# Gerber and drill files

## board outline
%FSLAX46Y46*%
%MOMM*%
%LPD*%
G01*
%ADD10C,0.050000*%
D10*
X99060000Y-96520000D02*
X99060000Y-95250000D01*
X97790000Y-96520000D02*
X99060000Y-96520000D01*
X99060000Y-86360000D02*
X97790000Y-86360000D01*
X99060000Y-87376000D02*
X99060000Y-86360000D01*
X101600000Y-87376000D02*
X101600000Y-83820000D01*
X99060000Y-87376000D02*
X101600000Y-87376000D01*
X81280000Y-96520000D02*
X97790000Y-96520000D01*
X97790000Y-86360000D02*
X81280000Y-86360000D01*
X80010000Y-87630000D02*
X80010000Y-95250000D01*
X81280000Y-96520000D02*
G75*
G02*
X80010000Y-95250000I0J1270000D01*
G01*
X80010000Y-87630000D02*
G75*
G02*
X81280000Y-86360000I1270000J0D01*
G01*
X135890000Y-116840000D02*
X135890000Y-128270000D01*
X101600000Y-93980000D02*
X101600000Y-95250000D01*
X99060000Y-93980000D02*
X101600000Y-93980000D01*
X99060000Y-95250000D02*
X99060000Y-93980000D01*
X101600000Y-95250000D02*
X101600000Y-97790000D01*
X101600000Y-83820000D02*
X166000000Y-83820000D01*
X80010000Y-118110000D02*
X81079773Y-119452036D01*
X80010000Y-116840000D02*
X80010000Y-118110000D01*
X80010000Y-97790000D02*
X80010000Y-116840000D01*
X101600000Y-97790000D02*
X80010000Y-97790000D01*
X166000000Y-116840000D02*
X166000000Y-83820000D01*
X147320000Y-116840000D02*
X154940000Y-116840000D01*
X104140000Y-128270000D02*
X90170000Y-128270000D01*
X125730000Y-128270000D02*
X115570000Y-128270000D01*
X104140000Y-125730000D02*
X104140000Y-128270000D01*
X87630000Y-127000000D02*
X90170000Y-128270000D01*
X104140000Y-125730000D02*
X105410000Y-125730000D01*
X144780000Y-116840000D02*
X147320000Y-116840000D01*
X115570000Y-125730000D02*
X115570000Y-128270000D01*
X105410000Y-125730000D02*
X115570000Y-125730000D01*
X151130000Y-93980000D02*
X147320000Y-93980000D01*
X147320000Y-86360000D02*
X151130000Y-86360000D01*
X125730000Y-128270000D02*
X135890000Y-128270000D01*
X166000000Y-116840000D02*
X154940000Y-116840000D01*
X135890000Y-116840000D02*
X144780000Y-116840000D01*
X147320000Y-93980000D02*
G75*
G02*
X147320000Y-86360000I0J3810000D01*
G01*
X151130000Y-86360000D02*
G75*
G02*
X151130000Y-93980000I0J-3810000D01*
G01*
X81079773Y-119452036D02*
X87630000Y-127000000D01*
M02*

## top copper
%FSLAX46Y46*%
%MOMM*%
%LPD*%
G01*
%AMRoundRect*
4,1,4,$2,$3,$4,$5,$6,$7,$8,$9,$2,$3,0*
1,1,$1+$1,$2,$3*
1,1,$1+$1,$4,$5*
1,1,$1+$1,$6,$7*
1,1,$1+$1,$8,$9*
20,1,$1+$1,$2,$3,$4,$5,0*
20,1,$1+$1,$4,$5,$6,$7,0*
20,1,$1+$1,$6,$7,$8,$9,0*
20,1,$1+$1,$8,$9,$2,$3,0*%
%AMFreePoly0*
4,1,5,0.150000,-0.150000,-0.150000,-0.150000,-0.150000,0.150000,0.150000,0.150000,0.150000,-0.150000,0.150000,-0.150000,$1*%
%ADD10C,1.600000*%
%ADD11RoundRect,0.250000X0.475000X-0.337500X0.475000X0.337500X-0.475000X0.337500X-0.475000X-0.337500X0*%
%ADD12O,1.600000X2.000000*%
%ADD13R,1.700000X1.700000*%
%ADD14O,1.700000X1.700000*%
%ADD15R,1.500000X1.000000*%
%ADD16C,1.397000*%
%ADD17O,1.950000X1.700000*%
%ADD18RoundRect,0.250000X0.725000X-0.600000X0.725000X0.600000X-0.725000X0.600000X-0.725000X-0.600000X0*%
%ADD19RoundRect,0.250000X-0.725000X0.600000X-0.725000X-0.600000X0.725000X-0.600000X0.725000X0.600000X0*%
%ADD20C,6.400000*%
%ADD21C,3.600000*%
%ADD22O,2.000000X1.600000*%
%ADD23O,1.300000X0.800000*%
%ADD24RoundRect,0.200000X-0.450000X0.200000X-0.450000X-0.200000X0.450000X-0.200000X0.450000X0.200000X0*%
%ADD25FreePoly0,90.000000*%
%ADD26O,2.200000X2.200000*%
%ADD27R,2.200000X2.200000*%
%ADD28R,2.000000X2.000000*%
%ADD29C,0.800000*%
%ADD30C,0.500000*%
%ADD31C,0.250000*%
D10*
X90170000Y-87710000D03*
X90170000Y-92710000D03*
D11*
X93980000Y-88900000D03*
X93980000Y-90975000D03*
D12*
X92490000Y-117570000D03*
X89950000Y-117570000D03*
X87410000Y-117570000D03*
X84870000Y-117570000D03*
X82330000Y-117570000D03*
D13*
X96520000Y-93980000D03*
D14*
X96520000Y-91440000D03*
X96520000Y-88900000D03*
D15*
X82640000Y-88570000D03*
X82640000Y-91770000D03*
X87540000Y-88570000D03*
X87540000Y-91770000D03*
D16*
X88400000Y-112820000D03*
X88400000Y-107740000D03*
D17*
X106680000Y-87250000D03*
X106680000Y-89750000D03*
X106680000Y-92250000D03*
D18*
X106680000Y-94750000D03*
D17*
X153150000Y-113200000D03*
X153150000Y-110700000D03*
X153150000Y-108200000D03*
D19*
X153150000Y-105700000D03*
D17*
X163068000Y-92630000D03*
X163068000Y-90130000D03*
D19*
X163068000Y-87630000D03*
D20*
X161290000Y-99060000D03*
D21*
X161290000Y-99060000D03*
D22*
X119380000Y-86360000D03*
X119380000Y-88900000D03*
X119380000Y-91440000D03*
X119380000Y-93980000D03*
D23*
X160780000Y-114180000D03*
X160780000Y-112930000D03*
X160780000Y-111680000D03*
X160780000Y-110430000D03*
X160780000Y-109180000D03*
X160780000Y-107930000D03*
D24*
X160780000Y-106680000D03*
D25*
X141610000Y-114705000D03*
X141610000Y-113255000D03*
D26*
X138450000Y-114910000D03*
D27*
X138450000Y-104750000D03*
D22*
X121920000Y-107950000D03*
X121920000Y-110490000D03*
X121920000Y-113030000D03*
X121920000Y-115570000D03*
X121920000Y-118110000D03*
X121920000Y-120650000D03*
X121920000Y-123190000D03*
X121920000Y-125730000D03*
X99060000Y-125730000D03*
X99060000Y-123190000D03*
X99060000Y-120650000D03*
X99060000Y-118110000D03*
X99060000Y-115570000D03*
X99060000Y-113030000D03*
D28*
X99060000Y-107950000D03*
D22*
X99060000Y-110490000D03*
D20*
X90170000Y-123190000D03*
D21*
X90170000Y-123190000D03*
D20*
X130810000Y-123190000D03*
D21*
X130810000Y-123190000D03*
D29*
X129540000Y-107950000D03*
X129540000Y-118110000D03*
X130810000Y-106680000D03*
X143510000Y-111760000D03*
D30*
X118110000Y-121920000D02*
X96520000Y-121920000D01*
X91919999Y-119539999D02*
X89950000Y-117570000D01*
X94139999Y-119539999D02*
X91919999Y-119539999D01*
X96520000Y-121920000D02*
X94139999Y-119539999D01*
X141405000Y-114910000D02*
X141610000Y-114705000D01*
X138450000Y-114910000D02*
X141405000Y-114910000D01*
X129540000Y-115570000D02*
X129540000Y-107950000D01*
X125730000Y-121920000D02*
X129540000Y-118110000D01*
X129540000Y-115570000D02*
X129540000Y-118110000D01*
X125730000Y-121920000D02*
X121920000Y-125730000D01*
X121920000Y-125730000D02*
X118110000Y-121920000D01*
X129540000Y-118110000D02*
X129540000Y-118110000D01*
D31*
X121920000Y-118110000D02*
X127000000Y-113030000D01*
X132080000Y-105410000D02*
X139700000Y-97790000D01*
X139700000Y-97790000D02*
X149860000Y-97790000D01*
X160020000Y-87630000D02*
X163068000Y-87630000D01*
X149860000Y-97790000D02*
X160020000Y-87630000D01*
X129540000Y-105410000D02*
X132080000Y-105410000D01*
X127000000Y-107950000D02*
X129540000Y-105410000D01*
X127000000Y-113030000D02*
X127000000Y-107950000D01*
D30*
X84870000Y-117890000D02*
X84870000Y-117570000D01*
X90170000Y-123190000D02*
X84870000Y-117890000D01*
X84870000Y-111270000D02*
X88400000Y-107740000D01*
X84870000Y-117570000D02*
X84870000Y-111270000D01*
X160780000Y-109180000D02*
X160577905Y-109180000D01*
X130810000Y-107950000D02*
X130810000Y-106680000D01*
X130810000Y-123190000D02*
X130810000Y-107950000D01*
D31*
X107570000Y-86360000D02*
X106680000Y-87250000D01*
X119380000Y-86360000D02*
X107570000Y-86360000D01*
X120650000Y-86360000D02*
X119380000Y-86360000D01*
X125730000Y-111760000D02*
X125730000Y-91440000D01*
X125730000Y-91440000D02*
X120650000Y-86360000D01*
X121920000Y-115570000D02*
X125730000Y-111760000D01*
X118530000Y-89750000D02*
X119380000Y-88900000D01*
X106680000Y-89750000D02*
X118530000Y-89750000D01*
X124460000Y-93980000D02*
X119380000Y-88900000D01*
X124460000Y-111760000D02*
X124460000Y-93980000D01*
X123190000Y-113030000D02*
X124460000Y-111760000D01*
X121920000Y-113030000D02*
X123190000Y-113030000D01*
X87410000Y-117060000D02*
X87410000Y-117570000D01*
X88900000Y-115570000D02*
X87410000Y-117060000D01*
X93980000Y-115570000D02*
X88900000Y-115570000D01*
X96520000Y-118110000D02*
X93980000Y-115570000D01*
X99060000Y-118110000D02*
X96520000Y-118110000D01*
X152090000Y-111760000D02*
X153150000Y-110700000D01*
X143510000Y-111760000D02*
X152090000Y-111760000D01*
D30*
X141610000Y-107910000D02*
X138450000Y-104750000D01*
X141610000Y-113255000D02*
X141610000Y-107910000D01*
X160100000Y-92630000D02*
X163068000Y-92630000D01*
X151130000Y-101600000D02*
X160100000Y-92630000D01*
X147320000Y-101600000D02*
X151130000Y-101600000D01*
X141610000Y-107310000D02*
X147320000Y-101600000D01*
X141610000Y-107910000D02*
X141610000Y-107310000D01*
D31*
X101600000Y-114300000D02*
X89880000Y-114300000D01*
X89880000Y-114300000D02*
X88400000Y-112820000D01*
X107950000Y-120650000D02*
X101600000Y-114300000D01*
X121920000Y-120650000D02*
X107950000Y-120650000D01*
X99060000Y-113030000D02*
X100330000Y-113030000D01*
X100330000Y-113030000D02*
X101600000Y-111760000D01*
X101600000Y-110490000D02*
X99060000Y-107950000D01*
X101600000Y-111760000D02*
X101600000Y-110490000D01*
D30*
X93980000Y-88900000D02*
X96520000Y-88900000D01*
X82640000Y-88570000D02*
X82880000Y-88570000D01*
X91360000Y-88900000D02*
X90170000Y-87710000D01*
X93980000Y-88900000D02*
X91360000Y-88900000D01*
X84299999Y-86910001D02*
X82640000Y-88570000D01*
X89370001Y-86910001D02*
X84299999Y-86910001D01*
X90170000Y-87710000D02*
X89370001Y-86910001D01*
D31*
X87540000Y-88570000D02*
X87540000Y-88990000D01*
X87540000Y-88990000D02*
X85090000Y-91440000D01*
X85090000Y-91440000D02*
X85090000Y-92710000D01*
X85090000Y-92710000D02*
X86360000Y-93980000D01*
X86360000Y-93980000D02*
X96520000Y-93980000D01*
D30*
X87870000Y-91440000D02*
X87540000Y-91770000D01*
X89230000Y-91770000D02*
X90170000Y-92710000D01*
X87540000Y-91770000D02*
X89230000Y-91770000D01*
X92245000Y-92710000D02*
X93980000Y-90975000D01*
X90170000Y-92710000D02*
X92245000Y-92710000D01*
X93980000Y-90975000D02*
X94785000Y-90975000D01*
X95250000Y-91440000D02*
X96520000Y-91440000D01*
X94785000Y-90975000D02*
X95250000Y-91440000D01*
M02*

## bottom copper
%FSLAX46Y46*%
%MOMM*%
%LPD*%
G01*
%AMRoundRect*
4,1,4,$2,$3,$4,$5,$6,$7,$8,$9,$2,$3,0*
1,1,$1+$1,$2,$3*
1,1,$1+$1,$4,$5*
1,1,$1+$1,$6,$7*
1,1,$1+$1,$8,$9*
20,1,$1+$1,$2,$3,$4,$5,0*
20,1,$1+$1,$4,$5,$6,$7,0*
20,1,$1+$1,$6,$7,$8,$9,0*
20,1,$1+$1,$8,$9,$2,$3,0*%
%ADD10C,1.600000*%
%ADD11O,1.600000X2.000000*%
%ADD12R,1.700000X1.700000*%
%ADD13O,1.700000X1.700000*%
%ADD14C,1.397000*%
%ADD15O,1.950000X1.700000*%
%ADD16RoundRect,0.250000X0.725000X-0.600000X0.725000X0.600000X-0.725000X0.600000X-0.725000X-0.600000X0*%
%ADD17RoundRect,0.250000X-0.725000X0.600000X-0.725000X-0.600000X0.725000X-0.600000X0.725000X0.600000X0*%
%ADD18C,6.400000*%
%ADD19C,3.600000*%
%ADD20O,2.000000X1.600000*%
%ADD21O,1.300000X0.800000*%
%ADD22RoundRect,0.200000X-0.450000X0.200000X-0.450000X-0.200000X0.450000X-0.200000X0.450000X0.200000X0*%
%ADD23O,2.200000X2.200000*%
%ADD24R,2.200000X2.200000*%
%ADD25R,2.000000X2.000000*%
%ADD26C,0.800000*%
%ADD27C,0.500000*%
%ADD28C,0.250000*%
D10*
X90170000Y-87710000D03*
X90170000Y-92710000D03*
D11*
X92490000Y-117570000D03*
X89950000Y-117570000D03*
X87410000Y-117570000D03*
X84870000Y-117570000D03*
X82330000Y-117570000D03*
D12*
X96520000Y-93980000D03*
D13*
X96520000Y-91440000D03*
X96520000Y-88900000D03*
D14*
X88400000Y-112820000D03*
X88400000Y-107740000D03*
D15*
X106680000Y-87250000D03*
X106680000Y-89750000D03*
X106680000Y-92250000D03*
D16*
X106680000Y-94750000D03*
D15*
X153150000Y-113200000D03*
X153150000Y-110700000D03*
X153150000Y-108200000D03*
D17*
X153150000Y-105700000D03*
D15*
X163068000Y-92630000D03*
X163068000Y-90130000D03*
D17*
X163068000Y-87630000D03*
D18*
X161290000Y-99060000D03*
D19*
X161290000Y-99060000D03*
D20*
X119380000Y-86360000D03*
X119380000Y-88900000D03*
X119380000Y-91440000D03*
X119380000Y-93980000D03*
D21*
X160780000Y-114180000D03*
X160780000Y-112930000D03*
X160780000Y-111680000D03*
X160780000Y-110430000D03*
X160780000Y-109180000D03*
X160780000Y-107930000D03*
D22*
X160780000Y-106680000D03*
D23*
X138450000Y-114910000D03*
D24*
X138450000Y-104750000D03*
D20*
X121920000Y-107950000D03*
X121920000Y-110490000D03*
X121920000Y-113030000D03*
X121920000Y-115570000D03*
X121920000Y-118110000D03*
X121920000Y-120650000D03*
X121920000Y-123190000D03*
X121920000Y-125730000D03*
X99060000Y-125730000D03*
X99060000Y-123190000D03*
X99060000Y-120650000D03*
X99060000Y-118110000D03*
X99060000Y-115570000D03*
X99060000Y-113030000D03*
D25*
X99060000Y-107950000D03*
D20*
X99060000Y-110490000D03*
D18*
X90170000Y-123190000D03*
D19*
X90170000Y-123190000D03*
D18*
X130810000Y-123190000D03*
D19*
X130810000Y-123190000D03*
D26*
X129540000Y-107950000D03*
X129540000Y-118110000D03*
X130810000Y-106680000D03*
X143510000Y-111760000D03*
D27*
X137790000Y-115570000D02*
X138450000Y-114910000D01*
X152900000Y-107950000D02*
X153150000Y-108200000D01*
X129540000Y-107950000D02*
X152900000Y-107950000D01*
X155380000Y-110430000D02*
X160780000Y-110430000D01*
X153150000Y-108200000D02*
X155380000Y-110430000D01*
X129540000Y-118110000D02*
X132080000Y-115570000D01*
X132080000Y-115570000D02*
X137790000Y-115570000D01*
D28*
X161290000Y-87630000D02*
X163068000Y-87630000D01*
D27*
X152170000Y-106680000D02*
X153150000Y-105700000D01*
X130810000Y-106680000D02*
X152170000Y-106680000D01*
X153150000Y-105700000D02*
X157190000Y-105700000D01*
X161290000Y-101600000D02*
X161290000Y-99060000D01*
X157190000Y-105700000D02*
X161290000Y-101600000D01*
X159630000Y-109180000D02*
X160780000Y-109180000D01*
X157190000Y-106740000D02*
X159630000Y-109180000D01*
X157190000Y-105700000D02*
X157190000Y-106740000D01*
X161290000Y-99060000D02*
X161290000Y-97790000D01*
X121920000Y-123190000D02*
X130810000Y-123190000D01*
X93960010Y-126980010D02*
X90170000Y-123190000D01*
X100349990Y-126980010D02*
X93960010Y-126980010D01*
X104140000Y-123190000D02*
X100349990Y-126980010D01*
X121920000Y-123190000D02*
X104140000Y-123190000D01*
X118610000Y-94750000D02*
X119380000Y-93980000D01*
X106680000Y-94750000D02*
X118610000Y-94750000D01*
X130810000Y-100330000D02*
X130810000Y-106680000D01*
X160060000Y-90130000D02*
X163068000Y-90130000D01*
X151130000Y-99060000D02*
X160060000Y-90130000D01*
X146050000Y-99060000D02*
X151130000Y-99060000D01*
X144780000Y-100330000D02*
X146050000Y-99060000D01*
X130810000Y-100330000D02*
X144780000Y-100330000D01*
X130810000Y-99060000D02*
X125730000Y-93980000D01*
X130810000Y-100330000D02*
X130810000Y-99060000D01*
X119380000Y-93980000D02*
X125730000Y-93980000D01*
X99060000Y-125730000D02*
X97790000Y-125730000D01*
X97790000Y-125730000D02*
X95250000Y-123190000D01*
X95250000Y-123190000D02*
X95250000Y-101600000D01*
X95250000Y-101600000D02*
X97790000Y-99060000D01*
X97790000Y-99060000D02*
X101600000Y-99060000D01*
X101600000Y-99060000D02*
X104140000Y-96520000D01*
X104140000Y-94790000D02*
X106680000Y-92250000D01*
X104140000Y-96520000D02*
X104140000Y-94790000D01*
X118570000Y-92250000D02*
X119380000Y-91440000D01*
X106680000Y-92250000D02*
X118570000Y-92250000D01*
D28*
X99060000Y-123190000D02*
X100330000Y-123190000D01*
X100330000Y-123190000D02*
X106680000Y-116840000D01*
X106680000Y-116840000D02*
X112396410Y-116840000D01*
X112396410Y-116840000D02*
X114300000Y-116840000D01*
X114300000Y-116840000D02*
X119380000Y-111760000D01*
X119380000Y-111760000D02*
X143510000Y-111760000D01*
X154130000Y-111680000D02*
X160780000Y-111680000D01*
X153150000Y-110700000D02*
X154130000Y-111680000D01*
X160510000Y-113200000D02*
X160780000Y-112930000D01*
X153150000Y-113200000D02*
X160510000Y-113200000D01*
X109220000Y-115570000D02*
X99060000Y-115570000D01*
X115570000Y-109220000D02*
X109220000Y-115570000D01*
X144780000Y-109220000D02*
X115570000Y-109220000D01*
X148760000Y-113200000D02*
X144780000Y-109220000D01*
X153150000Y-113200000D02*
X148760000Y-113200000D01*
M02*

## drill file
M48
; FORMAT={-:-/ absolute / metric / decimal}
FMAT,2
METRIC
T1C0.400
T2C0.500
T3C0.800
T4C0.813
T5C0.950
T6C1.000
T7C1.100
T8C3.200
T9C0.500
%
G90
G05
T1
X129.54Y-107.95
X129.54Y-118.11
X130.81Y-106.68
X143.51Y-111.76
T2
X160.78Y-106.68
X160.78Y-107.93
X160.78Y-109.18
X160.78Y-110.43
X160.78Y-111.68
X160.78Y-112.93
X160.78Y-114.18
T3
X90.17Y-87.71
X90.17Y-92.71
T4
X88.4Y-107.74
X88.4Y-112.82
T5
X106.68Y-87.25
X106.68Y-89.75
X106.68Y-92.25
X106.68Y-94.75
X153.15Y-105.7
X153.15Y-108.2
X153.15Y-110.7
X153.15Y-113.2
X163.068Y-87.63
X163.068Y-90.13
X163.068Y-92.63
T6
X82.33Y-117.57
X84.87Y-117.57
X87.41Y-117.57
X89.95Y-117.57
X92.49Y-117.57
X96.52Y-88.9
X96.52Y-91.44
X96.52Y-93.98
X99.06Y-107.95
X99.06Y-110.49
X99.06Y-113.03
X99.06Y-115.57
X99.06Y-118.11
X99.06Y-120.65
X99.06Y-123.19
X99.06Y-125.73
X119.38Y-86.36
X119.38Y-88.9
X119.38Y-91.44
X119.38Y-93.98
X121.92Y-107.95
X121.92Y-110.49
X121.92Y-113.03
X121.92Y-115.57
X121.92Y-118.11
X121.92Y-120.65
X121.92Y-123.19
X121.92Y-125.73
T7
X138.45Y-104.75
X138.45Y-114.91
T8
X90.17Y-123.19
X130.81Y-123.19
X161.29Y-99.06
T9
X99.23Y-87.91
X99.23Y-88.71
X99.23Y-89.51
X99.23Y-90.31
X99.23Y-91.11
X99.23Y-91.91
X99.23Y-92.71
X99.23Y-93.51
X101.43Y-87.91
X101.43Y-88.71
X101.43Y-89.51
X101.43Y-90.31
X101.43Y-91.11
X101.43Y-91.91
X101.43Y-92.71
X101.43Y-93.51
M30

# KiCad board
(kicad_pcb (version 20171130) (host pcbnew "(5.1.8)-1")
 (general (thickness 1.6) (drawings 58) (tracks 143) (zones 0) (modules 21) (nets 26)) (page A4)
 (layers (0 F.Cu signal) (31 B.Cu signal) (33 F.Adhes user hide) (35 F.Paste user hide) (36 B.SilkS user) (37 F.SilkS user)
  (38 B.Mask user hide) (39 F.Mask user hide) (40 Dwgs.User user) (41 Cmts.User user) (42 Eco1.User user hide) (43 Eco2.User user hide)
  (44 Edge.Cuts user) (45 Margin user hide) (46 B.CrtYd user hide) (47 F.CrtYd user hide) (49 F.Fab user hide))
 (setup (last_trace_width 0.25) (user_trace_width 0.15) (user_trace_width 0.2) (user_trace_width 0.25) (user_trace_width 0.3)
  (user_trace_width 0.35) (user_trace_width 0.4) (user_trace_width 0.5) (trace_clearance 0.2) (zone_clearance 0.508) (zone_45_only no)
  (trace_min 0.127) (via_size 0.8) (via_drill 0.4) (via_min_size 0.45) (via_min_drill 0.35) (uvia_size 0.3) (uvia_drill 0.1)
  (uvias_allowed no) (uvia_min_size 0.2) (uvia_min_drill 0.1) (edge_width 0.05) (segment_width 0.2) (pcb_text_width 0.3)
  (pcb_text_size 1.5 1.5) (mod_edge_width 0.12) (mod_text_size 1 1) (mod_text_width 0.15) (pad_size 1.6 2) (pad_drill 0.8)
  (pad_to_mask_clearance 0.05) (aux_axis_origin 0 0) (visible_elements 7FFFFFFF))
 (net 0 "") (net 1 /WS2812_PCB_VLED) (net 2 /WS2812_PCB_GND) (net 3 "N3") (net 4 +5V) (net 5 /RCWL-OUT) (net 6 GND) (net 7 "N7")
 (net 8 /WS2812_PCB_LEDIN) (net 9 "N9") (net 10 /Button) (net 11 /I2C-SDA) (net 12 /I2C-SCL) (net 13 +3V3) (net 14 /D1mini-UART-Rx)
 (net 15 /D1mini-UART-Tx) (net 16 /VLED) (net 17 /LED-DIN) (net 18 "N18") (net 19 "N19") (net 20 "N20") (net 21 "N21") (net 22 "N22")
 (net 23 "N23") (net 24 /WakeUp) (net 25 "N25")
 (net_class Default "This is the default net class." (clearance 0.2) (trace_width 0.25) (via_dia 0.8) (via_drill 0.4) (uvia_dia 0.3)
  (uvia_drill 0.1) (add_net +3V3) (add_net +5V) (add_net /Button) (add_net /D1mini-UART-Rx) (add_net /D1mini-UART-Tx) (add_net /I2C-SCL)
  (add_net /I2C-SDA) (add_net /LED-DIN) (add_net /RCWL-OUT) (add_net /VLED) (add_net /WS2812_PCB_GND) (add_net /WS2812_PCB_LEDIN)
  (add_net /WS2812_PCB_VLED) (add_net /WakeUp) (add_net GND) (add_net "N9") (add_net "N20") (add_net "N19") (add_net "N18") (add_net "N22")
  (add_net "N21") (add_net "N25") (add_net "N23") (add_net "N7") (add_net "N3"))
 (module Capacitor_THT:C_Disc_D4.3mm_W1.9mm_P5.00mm (layer F.Cu) (at 90.17 92.71 90)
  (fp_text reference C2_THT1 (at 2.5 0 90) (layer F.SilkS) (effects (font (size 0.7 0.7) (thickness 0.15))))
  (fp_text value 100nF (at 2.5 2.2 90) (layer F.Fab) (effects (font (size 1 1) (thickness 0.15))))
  (pad 2 thru_hole circle (at 5 0 90) (size 1.6 1.6) (drill 0.8) (layers *.Cu *.Mask) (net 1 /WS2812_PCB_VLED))
  (pad 1 thru_hole circle (at 0 0 90) (size 1.6 1.6) (drill 0.8) (layers *.Cu *.Mask) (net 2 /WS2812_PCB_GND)))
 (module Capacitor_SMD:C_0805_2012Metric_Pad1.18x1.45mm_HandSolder (layer F.Cu) (at 93.98 89.9375 90)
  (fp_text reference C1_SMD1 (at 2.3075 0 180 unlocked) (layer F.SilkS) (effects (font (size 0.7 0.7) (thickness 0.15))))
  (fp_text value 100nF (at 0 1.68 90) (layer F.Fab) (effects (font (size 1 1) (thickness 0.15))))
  (pad 2 smd roundrect (at 1.0375 0 90) (size 1.175 1.45) (layers F.Cu F.Paste F.Mask) (roundrect_rratio 0.2127659574468085)
   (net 1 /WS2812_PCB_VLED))
  (pad 1 smd roundrect (at -1.0375 0 90) (size 1.175 1.45) (layers F.Cu F.Paste F.Mask) (roundrect_rratio 0.2127659574468085)
   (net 2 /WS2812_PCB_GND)))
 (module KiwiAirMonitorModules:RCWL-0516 (layer F.Cu) (at 87.41 117.57)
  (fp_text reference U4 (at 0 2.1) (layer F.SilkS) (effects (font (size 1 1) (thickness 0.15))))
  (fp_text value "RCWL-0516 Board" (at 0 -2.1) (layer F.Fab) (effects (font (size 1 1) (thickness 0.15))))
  (pad 5 thru_hole oval (at 5.08 0) (size 1.6 2) (drill 1) (layers *.Cu *.Mask) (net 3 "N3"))
  (pad 4 thru_hole oval (at 2.54 0) (size 1.6 2) (drill 1) (layers *.Cu *.Mask) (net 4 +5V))
  (pad 3 thru_hole oval (at 0 0) (size 1.6 2) (drill 1) (layers *.Cu *.Mask) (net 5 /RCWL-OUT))
  (pad 2 thru_hole oval (at -2.54 0) (size 1.6 2) (drill 1) (layers *.Cu *.Mask) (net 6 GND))
  (pad 1 thru_hole oval (at -5.08 0) (size 1.6 2) (drill 1) (layers *.Cu *.Mask) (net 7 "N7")))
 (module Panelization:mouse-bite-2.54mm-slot (layer F.Cu) (at 100.33 92.71 90)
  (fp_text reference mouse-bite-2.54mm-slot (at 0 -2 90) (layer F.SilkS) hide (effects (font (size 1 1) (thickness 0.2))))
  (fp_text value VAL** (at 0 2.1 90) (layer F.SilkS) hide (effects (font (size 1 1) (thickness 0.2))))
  (pad "" np_thru_hole circle (at 0.8 1.1 90) (size 0.5 0.5) (drill 0.5) (layers *.Cu *.Mask))
  (pad "" np_thru_hole circle (at -0.8 1.1 90) (size 0.5 0.5) (drill 0.5) (layers *.Cu *.Mask))
  (pad "" np_thru_hole circle (at -0.8 -1.1 90) (size 0.5 0.5) (drill 0.5) (layers *.Cu *.Mask))
  (pad "" np_thru_hole circle (at 0.8 -1.1 90) (size 0.5 0.5) (drill 0.5) (layers *.Cu *.Mask))
  (pad "" np_thru_hole circle (at 0 1.1 90) (size 0.5 0.5) (drill 0.5) (layers *.Cu *.Mask))
  (pad "" np_thru_hole circle (at 0 -1.1 90) (size 0.5 0.5) (drill 0.5) (layers *.Cu *.Mask))
  (pad "" np_thru_hole circle (at 1.6 -1.1 90) (size 0.5 0.5) (drill 0.5) (layers *.Cu *.Mask))
  (pad "" np_thru_hole circle (at 2.4 -1.1 90) (size 0.5 0.5) (drill 0.5) (layers *.Cu *.Mask))
  (pad "" np_thru_hole circle (at 3.2 -1.1 90) (size 0.5 0.5) (drill 0.5) (layers *.Cu *.Mask))
  (pad "" np_thru_hole circle (at 1.6 1.1 90) (size 0.5 0.5) (drill 0.5) (layers *.Cu *.Mask))
  (pad "" np_thru_hole circle (at 2.4 1.1 90) (size 0.5 0.5) (drill 0.5) (layers *.Cu *.Mask))
  (pad "" np_thru_hole circle (at 3.2 1.1 90) (size 0.5 0.5) (drill 0.5) (layers *.Cu *.Mask))
  (pad "" np_thru_hole circle (at 4 -1.1 90) (size 0.5 0.5) (drill 0.5) (layers *.Cu *.Mask))
  (pad "" np_thru_hole circle (at 4 1.1 90) (size 0.5 0.5) (drill 0.5) (layers *.Cu *.Mask))
  (pad "" np_thru_hole circle (at 4.8 -1.1 90) (size 0.5 0.5) (drill 0.5) (layers *.Cu *.Mask))
  (pad "" np_thru_hole circle (at 4.8 1.1 90) (size 0.5 0.5) (drill 0.5) (layers *.Cu *.Mask)))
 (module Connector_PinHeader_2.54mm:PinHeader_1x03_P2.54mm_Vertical (layer B.Cu) (at 96.52 93.98)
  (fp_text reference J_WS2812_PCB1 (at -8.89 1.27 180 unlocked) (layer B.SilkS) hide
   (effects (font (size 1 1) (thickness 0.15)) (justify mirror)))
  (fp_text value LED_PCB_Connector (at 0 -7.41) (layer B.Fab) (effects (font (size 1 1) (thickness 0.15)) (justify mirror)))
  (pad 1 thru_hole rect (at 0 0) (size 1.7 1.7) (drill 1) (layers *.Cu *.Mask) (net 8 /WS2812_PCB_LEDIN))
  (pad 2 thru_hole oval (at 0 -2.54) (size 1.7 1.7) (drill 1) (layers *.Cu *.Mask) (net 2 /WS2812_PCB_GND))
  (pad 3 thru_hole oval (at 0 -5.08) (size 1.7 1.7) (drill 1) (layers *.Cu *.Mask) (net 1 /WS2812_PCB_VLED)))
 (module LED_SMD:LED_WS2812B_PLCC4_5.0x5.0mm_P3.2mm (layer F.Cu) (at 85.09 90.17)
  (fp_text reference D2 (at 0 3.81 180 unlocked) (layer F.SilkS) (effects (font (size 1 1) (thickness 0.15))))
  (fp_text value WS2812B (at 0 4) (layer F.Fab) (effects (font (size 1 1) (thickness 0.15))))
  (pad 1 smd rect (at -2.45 -1.6) (size 1.5 1) (layers F.Cu F.Paste F.Mask) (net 1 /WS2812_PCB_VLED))
  (pad 2 smd rect (at -2.45 1.6) (size 1.5 1) (layers F.Cu F.Paste F.Mask) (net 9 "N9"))
  (pad 4 smd rect (at 2.45 -1.6) (size 1.5 1) (layers F.Cu F.Paste F.Mask) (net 8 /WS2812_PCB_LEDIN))
  (pad 3 smd rect (at 2.45 1.6) (size 1.5 1) (layers F.Cu F.Paste F.Mask) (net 2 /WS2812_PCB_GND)))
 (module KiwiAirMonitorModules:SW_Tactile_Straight (layer B.Cu) (at 88.4 112.82)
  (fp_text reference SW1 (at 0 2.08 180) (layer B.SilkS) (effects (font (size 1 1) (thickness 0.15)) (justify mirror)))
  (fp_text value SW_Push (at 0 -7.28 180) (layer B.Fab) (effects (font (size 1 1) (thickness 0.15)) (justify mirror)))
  (pad 1 thru_hole circle (at 0 0) (size 1.397 1.397) (drill 0.8128) (layers *.Cu *.Mask) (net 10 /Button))
  (pad 2 thru_hole circle (at 0 -5.08) (size 1.397 1.397) (drill 0.8128) (layers *.Cu *.Mask) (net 6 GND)))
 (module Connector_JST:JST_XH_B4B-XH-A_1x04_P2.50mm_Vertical (layer F.Cu) (at 106.68 94.75 90)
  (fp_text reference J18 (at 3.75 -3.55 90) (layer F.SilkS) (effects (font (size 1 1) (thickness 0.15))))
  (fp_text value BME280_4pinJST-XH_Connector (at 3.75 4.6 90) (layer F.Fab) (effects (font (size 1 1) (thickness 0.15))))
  (pad 4 thru_hole oval (at 7.5 0 90) (size 1.7 1.95) (drill 0.95) (layers *.Cu *.Mask) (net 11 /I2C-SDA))
  (pad 3 thru_hole oval (at 5 0 90) (size 1.7 1.95) (drill 0.95) (layers *.Cu *.Mask) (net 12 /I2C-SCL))
  (pad 2 thru_hole oval (at 2.5 0 90) (size 1.7 1.95) (drill 0.95) (layers *.Cu *.Mask) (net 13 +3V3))
  (pad 1 thru_hole roundrect (at 0 0 90) (size 1.7 1.95) (drill 0.95) (layers *.Cu *.Mask) (roundrect_rratio 0.1470588235294118) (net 6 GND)))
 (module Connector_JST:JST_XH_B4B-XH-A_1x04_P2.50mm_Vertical (layer F.Cu) (at 153.15 105.7 270)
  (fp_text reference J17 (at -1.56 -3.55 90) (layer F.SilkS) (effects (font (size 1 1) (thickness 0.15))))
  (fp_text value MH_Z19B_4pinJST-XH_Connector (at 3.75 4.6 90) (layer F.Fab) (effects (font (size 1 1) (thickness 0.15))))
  (pad 4 thru_hole oval (at 7.5 0 270) (size 1.7 1.95) (drill 0.95) (layers *.Cu *.Mask) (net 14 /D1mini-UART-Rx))
  (pad 3 thru_hole oval (at 5 0 270) (size 1.7 1.95) (drill 0.95) (layers *.Cu *.Mask) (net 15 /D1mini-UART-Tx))
  (pad 2 thru_hole oval (at 2.5 0 270) (size 1.7 1.95) (drill 0.95) (layers *.Cu *.Mask) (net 4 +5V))
  (pad 1 thru_hole roundrect (at 0 0 270) (size 1.7 1.95) (drill 0.95) (layers *.Cu *.Mask) (roundrect_rratio 0.1470588235294118)
   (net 6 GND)))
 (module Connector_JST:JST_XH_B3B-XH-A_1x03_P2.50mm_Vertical (layer F.Cu) (at 163.068 87.63 270)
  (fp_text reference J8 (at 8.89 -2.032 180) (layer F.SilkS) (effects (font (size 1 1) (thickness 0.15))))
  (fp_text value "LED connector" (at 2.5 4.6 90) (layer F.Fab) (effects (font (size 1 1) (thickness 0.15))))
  (pad 3 thru_hole oval (at 5 0 270) (size 1.7 1.95) (drill 0.95) (layers *.Cu *.Mask) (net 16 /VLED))
  (pad 2 thru_hole oval (at 2.5 0 270) (size 1.7 1.95) (drill 0.95) (layers *.Cu *.Mask) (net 6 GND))
  (pad 1 thru_hole roundrect (at 0 0 270) (size 1.7 1.95) (drill 0.95) (layers *.Cu *.Mask) (roundrect_rratio 0.1470588235294118)
   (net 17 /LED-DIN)))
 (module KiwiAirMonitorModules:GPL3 (layer B.Cu) (at 132.08 90.17 180)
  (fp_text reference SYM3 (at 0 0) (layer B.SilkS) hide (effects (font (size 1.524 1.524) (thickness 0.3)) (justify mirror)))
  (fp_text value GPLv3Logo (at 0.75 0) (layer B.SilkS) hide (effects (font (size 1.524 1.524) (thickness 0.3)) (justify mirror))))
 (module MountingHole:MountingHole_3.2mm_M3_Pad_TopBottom (layer F.Cu) (at 161.29 99.06)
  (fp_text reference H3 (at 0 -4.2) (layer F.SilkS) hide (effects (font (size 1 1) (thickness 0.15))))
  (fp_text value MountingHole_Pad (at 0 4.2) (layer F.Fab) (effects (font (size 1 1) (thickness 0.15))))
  (pad 1 connect circle (at 0 0) (size 6.4 6.4) (layers B.Cu B.Mask) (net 6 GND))
  (pad 1 connect circle (at 0 0) (size 6.4 6.4) (layers F.Cu F.Mask) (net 6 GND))
  (pad 1 thru_hole circle (at 0 0) (size 3.6 3.6) (drill 3.2) (layers *.Cu *.Mask) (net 6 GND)))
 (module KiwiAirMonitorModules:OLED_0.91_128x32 (layer F.Cu) (at 119.38 90.17 270)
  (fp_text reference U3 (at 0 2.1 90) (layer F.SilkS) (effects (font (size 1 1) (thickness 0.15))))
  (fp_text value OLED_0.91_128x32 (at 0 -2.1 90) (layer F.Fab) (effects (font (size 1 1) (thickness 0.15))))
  (pad 4 thru_hole oval (at -3.81 0 270) (size 1.6 2) (drill 1) (layers *.Cu *.Mask) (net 11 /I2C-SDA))
  (pad 3 thru_hole oval (at -1.27 0 270) (size 1.6 2) (drill 1) (layers *.Cu *.Mask) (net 12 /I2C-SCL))
  (pad 2 thru_hole oval (at 1.27 0 270) (size 1.6 2) (drill 1) (layers *.Cu *.Mask) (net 13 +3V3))
  (pad 1 thru_hole oval (at 3.81 0 270) (size 1.6 2) (drill 1) (layers *.Cu *.Mask) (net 6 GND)))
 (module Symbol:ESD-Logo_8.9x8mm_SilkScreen (layer F.Cu) (at 129.54 113.03)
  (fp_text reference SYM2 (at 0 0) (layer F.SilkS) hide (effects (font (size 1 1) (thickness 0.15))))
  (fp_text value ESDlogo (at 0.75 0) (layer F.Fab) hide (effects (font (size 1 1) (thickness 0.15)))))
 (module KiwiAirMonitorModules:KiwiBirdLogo (layer F.Cu) (at 130.81 101.6)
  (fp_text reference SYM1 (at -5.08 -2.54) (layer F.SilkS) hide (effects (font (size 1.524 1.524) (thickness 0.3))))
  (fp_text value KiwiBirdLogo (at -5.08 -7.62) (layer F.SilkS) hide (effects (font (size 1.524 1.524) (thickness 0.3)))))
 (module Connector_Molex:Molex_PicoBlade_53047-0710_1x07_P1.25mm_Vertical (layer F.Cu) (at 160.78 106.68 270)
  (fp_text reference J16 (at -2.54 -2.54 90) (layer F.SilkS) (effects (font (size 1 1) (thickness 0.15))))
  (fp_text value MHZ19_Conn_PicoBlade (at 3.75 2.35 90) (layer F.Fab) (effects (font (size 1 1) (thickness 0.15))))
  (pad 7 thru_hole oval (at 7.5 0 270) (size 0.8 1.3) (drill 0.5) (layers *.Cu *.Mask) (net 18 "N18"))
  (pad 6 thru_hole oval (at 6.25 0 270) (size 0.8 1.3) (drill 0.5) (layers *.Cu *.Mask) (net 14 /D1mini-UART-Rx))
  (pad 5 thru_hole oval (at 5 0 270) (size 0.8 1.3) (drill 0.5) (layers *.Cu *.Mask) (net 15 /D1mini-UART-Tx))
  (pad 4 thru_hole oval (at 3.75 0 270) (size 0.8 1.3) (drill 0.5) (layers *.Cu *.Mask) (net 4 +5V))
  (pad 3 thru_hole oval (at 2.5 0 270) (size 0.8 1.3) (drill 0.5) (layers *.Cu *.Mask) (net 6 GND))
  (pad 2 thru_hole oval (at 1.25 0 270) (size 0.8 1.3) (drill 0.5) (layers *.Cu *.Mask) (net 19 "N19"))
  (pad 1 thru_hole roundrect (at 0 0 270) (size 0.8 1.3) (drill 0.5) (layers *.Cu *.Mask) (roundrect_rratio 0.25) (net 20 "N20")))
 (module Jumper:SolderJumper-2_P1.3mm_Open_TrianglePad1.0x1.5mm (layer F.Cu) (at 141.61 113.98 90)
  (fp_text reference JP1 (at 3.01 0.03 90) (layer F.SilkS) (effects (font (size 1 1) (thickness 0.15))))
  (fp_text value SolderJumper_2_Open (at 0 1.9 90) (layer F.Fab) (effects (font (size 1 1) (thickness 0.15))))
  (pad 1 smd custom (at -0.725 0 90) (size 0.3 0.3) (layers F.Cu F.Mask) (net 4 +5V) (zone_connect 2)
   (options (clearance outline) (anchor rect)) (primitives))
  (pad 2 smd custom (at 0.725 0 90) (size 0.3 0.3) (layers F.Cu F.Mask) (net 16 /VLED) (zone_connect 2)
   (options (clearance outline) (anchor rect)) (primitives)))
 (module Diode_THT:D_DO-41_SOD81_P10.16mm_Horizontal (layer F.Cu) (at 138.45 104.75 270)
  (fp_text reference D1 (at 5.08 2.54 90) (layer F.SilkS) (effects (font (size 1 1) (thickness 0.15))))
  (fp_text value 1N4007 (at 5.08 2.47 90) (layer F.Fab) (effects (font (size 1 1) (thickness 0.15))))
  (pad 2 thru_hole oval (at 10.16 0 270) (size 2.2 2.2) (drill 1.1) (layers *.Cu *.Mask) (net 4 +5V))
  (pad 1 thru_hole rect (at 0 0 270) (size 2.2 2.2) (drill 1.1) (layers *.Cu *.Mask) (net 16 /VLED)))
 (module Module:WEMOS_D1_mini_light (layer F.Cu) (at 99.06 107.95)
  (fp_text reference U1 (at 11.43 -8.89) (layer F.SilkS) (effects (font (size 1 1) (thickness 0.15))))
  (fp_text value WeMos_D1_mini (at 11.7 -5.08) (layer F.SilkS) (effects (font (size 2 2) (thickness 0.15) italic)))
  (pad 16 thru_hole oval (at 22.86 0) (size 2 1.6) (drill 1) (layers *.Cu *.Mask) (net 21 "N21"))
  (pad 15 thru_hole oval (at 22.86 2.54) (size 2 1.6) (drill 1) (layers *.Cu *.Mask) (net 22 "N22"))
  (pad 14 thru_hole oval (at 22.86 5.08) (size 2 1.6) (drill 1) (layers *.Cu *.Mask) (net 12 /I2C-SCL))
  (pad 13 thru_hole oval (at 22.86 7.62) (size 2 1.6) (drill 1) (layers *.Cu *.Mask) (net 11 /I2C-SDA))
  (pad 12 thru_hole oval (at 22.86 10.16) (size 2 1.6) (drill 1) (layers *.Cu *.Mask) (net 17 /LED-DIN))
  (pad 11 thru_hole oval (at 22.86 12.7) (size 2 1.6) (drill 1) (layers *.Cu *.Mask) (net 10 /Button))
  (pad 10 thru_hole oval (at 22.86 15.24) (size 2 1.6) (drill 1) (layers *.Cu *.Mask) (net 6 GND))
  (pad 9 thru_hole oval (at 22.86 17.78) (size 2 1.6) (drill 1) (layers *.Cu *.Mask) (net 4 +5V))
  (pad 8 thru_hole oval (at 0 17.78) (size 2 1.6) (drill 1) (layers *.Cu *.Mask) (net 13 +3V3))
  (pad 7 thru_hole oval (at 0 15.24) (size 2 1.6) (drill 1) (layers *.Cu *.Mask) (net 15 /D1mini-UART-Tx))
  (pad 6 thru_hole oval (at 0 12.7) (size 2 1.6) (drill 1) (layers *.Cu *.Mask) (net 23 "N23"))
  (pad 5 thru_hole oval (at 0 10.16) (size 2 1.6) (drill 1) (layers *.Cu *.Mask) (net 5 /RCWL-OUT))
  (pad 4 thru_hole oval (at 0 7.62) (size 2 1.6) (drill 1) (layers *.Cu *.Mask) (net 14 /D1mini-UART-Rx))
  (pad 3 thru_hole oval (at 0 5.08) (size 2 1.6) (drill 1) (layers *.Cu *.Mask) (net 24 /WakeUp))
  (pad 1 thru_hole rect (at 0 0) (size 2 2) (drill 1) (layers *.Cu *.Mask) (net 24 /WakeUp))
  (pad 2 thru_hole oval (at 0 2.54) (size 2 1.6) (drill 1) (layers *.Cu *.Mask) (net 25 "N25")))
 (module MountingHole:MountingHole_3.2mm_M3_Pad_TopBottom (layer F.Cu) (at 90.17 123.19)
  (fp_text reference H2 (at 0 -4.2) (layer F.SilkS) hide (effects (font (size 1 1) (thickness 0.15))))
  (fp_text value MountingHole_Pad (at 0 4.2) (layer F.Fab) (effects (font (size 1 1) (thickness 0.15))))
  (pad 1 connect circle (at 0 0) (size 6.4 6.4) (layers B.Cu B.Mask) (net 6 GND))
  (pad 1 connect circle (at 0 0) (size 6.4 6.4) (layers F.Cu F.Mask) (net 6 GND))
  (pad 1 thru_hole circle (at 0 0) (size 3.6 3.6) (drill 3.2) (layers *.Cu *.Mask) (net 6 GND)))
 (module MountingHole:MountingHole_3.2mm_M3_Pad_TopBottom (layer F.Cu) (at 130.81 123.19)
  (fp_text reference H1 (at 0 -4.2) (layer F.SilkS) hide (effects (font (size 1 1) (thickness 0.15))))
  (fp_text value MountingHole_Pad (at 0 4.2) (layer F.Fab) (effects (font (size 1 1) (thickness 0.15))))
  (pad 1 connect circle (at 0 0) (size 6.4 6.4) (layers B.Cu B.Mask) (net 6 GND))
  (pad 1 connect circle (at 0 0) (size 6.4 6.4) (layers F.Cu F.Mask) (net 6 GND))
  (pad 1 thru_hole circle (at 0 0) (size 3.6 3.6) (drill 3.2) (layers *.Cu *.Mask) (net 6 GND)))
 (gr_line (start 99.06 96.52) (end 99.06 95.25) (layer Edge.Cuts) (width 0.05))
 (gr_line (start 97.79 96.52) (end 99.06 96.52) (layer Edge.Cuts) (width 0.05))
 (gr_line (start 99.06 86.36) (end 97.79 86.36) (layer Edge.Cuts) (width 0.05))
 (gr_line (start 99.06 87.376) (end 99.06 86.36) (layer Edge.Cuts) (width 0.05))
 (gr_line (start 101.6 87.376) (end 101.6 83.82) (layer Edge.Cuts) (width 0.05))
 (gr_line (start 99.06 87.376) (end 101.6 87.376) (layer Edge.Cuts) (width 0.05))
 (gr_line (start 81.28 96.52) (end 97.79 96.52) (layer Edge.Cuts) (width 0.05))
 (gr_line (start 97.79 86.36) (end 81.28 86.36) (layer Edge.Cuts) (width 0.05))
 (gr_line (start 80.01 87.63) (end 80.01 95.25) (layer Edge.Cuts) (width 0.05))
 (gr_arc (start 81.28 95.25) (end 80.01 95.25) (angle -90) (layer Edge.Cuts) (width 0.05))
 (gr_arc (start 81.28 87.63) (end 81.28 86.36) (angle -90) (layer Edge.Cuts) (width 0.05))
 (gr_line (start 135.89 116.84) (end 135.89 128.27) (layer Edge.Cuts) (width 0.05))
 (gr_line (start 101.6 93.98) (end 101.6 95.25) (layer Edge.Cuts) (width 0.05))
 (gr_line (start 99.06 93.98) (end 101.6 93.98) (layer Edge.Cuts) (width 0.05))
 (gr_line (start 99.06 95.25) (end 99.06 93.98) (layer Edge.Cuts) (width 0.05))
 (gr_line (start 101.6 95.25) (end 101.6 97.79) (layer Edge.Cuts) (width 0.05))
 (gr_line (start 101.6 83.82) (end 166 83.82) (layer Edge.Cuts) (width 0.05))
 (gr_line (start 80.01 118.11) (end 81.079773 119.452036) (layer Edge.Cuts) (width 0.05))
 (gr_line (start 80.01 116.84) (end 80.01 118.11) (layer Edge.Cuts) (width 0.05))
 (gr_line (start 80.01 97.79) (end 80.01 116.84) (layer Edge.Cuts) (width 0.05))
 (gr_line (start 101.6 97.79) (end 80.01 97.79) (layer Edge.Cuts) (width 0.05))
 (gr_line (start 166 116.84) (end 166 83.82) (layer Edge.Cuts) (width 0.05))
 (gr_line (start 147.32 116.84) (end 154.94 116.84) (layer Edge.Cuts) (width 0.05))
 (gr_line (start 104.14 128.27) (end 90.17 128.27) (layer Edge.Cuts) (width 0.05))
 (gr_line (start 125.73 128.27) (end 115.57 128.27) (layer Edge.Cuts) (width 0.05))
 (gr_line (start 104.14 125.73) (end 104.14 128.27) (layer Edge.Cuts) (width 0.05))
 (gr_line (start 87.63 127) (end 90.17 128.27) (layer Edge.Cuts) (width 0.05))
 (gr_line (start 104.14 125.73) (end 105.41 125.73) (layer Edge.Cuts) (width 0.05))
 (gr_line (start 144.78 116.84) (end 147.32 116.84) (layer Edge.Cuts) (width 0.05))
 (gr_line (start 115.57 125.73) (end 115.57 128.27) (layer Edge.Cuts) (width 0.05))
 (gr_line (start 105.41 125.73) (end 115.57 125.73) (layer Edge.Cuts) (width 0.05))
 (gr_line (start 151.13 93.98) (end 147.32 93.98) (layer Edge.Cuts) (width 0.05))
 (gr_line (start 147.32 86.36) (end 151.13 86.36) (layer Edge.Cuts) (width 0.05))
 (gr_line (start 125.73 128.27) (end 135.89 128.27) (layer Edge.Cuts) (width 0.05))
 (gr_line (start 166 116.84) (end 154.94 116.84) (layer Edge.Cuts) (width 0.05))
 (gr_line (start 135.89 116.84) (end 144.78 116.84) (layer Edge.Cuts) (width 0.05))
 (gr_arc (start 147.32 90.17) (end 147.32 86.36) (angle -180) (layer Edge.Cuts) (width 0.05))
 (gr_arc (start 151.13 90.17) (end 151.13 93.98) (angle -180) (layer Edge.Cuts) (width 0.05))
 (gr_line (start 81.079773 119.452036) (end 87.63 127) (layer Edge.Cuts) (width 0.05))
 (segment (start 118.11 121.92) (end 96.52 121.92) (width 0.5) (layer F.Cu) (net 4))
 (segment (start 91.919999 119.539999) (end 89.95 117.57) (width 0.5) (layer F.Cu) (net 4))
 (segment (start 94.139999 119.539999) (end 91.919999 119.539999) (width 0.5) (layer F.Cu) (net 4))
 (segment (start 96.52 121.92) (end 94.139999 119.539999) (width 0.5) (layer F.Cu) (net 4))
 (segment (start 137.79 115.57) (end 138.45 114.91) (width 0.5) (layer B.Cu) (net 4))
 (segment (start 141.405 114.91) (end 141.61 114.705) (width 0.5) (layer F.Cu) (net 4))
 (segment (start 138.45 114.91) (end 141.405 114.91) (width 0.5) (layer F.Cu) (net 4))
 (via (at 129.54 107.95) (size 0.8) (drill 0.4) (layers F.Cu B.Cu) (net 4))
 (segment (start 129.54 115.57) (end 129.54 107.95) (width 0.5) (layer F.Cu) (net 4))
 (segment (start 152.9 107.95) (end 153.15 108.2) (width 0.5) (layer B.Cu) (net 4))
 (segment (start 129.54 107.95) (end 152.9 107.95) (width 0.5) (layer B.Cu) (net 4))
 (segment (start 155.38 110.43) (end 160.78 110.43) (width 0.5) (layer B.Cu) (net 4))
 (segment (start 153.15 108.2) (end 155.38 110.43) (width 0.5) (layer B.Cu) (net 4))
 (segment (start 125.73 121.92) (end 129.54 118.11) (width 0.5) (layer F.Cu) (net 4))
 (segment (start 129.54 115.57) (end 129.54 118.11) (width 0.5) (layer F.Cu) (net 4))
 (segment (start 125.73 121.92) (end 121.92 125.73) (width 0.5) (layer F.Cu) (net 4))
 (segment (start 121.92 125.73) (end 118.11 121.92) (width 0.5) (layer F.Cu) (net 4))
 (segment (start 129.54 118.11) (end 129.54 118.11) (width 0.5) (layer F.Cu) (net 4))
 (via (at 129.54 118.11) (size 0.8) (drill 0.4) (layers F.Cu B.Cu) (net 4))
 (segment (start 129.54 118.11) (end 132.08 115.57) (width 0.5) (layer B.Cu) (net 4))
 (segment (start 132.08 115.57) (end 137.79 115.57) (width 0.5) (layer B.Cu) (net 4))
 (segment (start 121.92 118.11) (end 127 113.03) (width 0.25) (layer F.Cu) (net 17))
 (segment (start 161.29 87.63) (end 163.068 87.63) (width 0.25) (layer B.Cu) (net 17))
 (segment (start 132.08 105.41) (end 139.7 97.79) (width 0.25) (layer F.Cu) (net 17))
 (segment (start 139.7 97.79) (end 149.86 97.79) (width 0.25) (layer F.Cu) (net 17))
 (segment (start 160.02 87.63) (end 163.068 87.63) (width 0.25) (layer F.Cu) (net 17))
 (segment (start 149.86 97.79) (end 160.02 87.63) (width 0.25) (layer F.Cu) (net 17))
 (segment (start 129.54 105.41) (end 132.08 105.41) (width 0.25) (layer F.Cu) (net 17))
 (segment (start 127 107.95) (end 129.54 105.41) (width 0.25) (layer F.Cu) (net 17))
 (segment (start 127 113.03) (end 127 107.95) (width 0.25) (layer F.Cu) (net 17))
 (segment (start 84.87 117.89) (end 84.87 117.57) (width 0.5) (layer F.Cu) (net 6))
 (segment (start 90.17 123.19) (end 84.87 117.89) (width 0.5) (layer F.Cu) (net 6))
 (segment (start 84.87 111.27) (end 88.4 107.74) (width 0.5) (layer F.Cu) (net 6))
 (segment (start 84.87 117.57) (end 84.87 111.27) (width 0.5) (layer F.Cu) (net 6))
 (segment (start 160.78 109.18) (end 160.577905 109.18) (width 0.5) (layer F.Cu) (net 6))
 (segment (start 130.81 107.95) (end 130.81 106.68) (width 0.5) (layer F.Cu) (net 6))
 (segment (start 130.81 123.19) (end 130.81 107.95) (width 0.5) (layer F.Cu) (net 6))
 (via (at 130.81 106.68) (size 0.8) (drill 0.4) (layers F.Cu B.Cu) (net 6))
 (segment (start 152.17 106.68) (end 153.15 105.7) (width 0.5) (layer B.Cu) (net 6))
 (segment (start 130.81 106.68) (end 152.17 106.68) (width 0.5) (layer B.Cu) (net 6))
 (segment (start 153.15 105.7) (end 157.19 105.7) (width 0.5) (layer B.Cu) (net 6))
 (segment (start 161.29 101.6) (end 161.29 99.06) (width 0.5) (layer B.Cu) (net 6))
 (segment (start 157.19 105.7) (end 161.29 101.6) (width 0.5) (layer B.Cu) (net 6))
 (segment (start 159.63 109.18) (end 160.78 109.18) (width 0.5) (layer B.Cu) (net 6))
 (segment (start 157.19 106.74) (end 159.63 109.18) (width 0.5) (layer B.Cu) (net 6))
 (segment (start 157.19 105.7) (end 157.19 106.74) (width 0.5) (layer B.Cu) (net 6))
 (segment (start 161.29 99.06) (end 161.29 97.79) (width 0.5) (layer B.Cu) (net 6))
 (segment (start 121.92 123.19) (end 130.81 123.19) (width 0.5) (layer B.Cu) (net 6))
 (segment (start 93.96001 126.98001) (end 90.17 123.19) (width 0.5) (layer B.Cu) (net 6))
 (segment (start 100.34999 126.98001) (end 93.96001 126.98001) (width 0.5) (layer B.Cu) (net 6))
 (segment (start 104.14 123.19) (end 100.34999 126.98001) (width 0.5) (layer B.Cu) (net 6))
 (segment (start 121.92 123.19) (end 104.14 123.19) (width 0.5) (layer B.Cu) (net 6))
 (segment (start 118.61 94.75) (end 119.38 93.98) (width 0.5) (layer B.Cu) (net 6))
 (segment (start 106.68 94.75) (end 118.61 94.75) (width 0.5) (layer B.Cu) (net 6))
 (segment (start 130.81 100.33) (end 130.81 106.68) (width 0.5) (layer B.Cu) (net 6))
 (segment (start 160.06 90.13) (end 163.068 90.13) (width 0.5) (layer B.Cu) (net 6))
 (segment (start 151.13 99.06) (end 160.06 90.13) (width 0.5) (layer B.Cu) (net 6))
 (segment (start 146.05 99.06) (end 151.13 99.06) (width 0.5) (layer B.Cu) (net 6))
 (segment (start 144.78 100.33) (end 146.05 99.06) (width 0.5) (layer B.Cu) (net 6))
 (segment (start 130.81 100.33) (end 144.78 100.33) (width 0.5) (layer B.Cu) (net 6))
 (segment (start 130.81 99.06) (end 125.73 93.98) (width 0.5) (layer B.Cu) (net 6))
 (segment (start 130.81 100.33) (end 130.81 99.06) (width 0.5) (layer B.Cu) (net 6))
 (segment (start 119.38 93.98) (end 125.73 93.98) (width 0.5) (layer B.Cu) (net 6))
 (segment (start 107.57 86.36) (end 106.68 87.25) (width 0.25) (layer F.Cu) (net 11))
 (segment (start 119.38 86.36) (end 107.57 86.36) (width 0.25) (layer F.Cu) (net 11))
 (segment (start 120.65 86.36) (end 119.38 86.36) (width 0.25) (layer F.Cu) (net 11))
 (segment (start 125.73 111.76) (end 125.73 91.44) (width 0.25) (layer F.Cu) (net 11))
 (segment (start 125.73 91.44) (end 120.65 86.36) (width 0.25) (layer F.Cu) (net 11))
 (segment (start 121.92 115.57) (end 125.73 111.76) (width 0.25) (layer F.Cu) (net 11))
 (segment (start 118.53 89.75) (end 119.38 88.9) (width 0.25) (layer F.Cu) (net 12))
 (segment (start 106.68 89.75) (end 118.53 89.75) (width 0.25) (layer F.Cu) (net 12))
 (segment (start 124.46 93.98) (end 119.38 88.9) (width 0.25) (layer F.Cu) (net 12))
 (segment (start 124.46 111.76) (end 124.46 93.98) (width 0.25) (layer F.Cu) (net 12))
 (segment (start 123.19 113.03) (end 124.46 111.76) (width 0.25) (layer F.Cu) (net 12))
 (segment (start 121.92 113.03) (end 123.19 113.03) (width 0.25) (layer F.Cu) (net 12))
 (segment (start 87.41 117.06) (end 87.41 117.57) (width 0.25) (layer F.Cu) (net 5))
 (segment (start 88.9 115.57) (end 87.41 117.06) (width 0.25) (layer F.Cu) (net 5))
 (segment (start 93.98 115.57) (end 88.9 115.57) (width 0.25) (layer F.Cu) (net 5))
 (segment (start 96.52 118.11) (end 93.98 115.57) (width 0.25) (layer F.Cu) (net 5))
 (segment (start 99.06 118.11) (end 96.52 118.11) (width 0.25) (layer F.Cu) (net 5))
 (segment (start 99.06 125.73) (end 97.79 125.73) (width 0.5) (layer B.Cu) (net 13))
 (segment (start 97.79 125.73) (end 95.25 123.19) (width 0.5) (layer B.Cu) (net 13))
 (segment (start 95.25 123.19) (end 95.25 101.6) (width 0.5) (layer B.Cu) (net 13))
 (segment (start 95.25 101.6) (end 97.79 99.06) (width 0.5) (layer B.Cu) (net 13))
 (segment (start 97.79 99.06) (end 101.6 99.06) (width 0.5) (layer B.Cu) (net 13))
 (segment (start 101.6 99.06) (end 104.14 96.52) (width 0.5) (layer B.Cu) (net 13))
 (segment (start 104.14 94.79) (end 106.68 92.25) (width 0.5) (layer B.Cu) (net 13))
 (segment (start 104.14 96.52) (end 104.14 94.79) (width 0.5) (layer B.Cu) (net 13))
 (segment (start 118.57 92.25) (end 119.38 91.44) (width 0.5) (layer B.Cu) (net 13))
 (segment (start 106.68 92.25) (end 118.57 92.25) (width 0.5) (layer B.Cu) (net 13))
 (segment (start 99.06 123.19) (end 100.33 123.19) (width 0.25) (layer B.Cu) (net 15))
 (segment (start 100.33 123.19) (end 106.68 116.84) (width 0.25) (layer B.Cu) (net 15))
 (segment (start 106.68 116.84) (end 112.39641 116.84) (width 0.25) (layer B.Cu) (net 15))
 (segment (start 112.39641 116.84) (end 114.3 116.84) (width 0.25) (layer B.Cu) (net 15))
 (segment (start 114.3 116.84) (end 119.38 111.76) (width 0.25) (layer B.Cu) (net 15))
 (via (at 143.51 111.76) (size 0.8) (drill 0.4) (layers F.Cu B.Cu) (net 15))
 (segment (start 119.38 111.76) (end 143.51 111.76) (width 0.25) (layer B.Cu) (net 15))
 (segment (start 152.09 111.76) (end 153.15 110.7) (width 0.25) (layer F.Cu) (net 15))
 (segment (start 143.51 111.76) (end 152.09 111.76) (width 0.25) (layer F.Cu) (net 15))
 (segment (start 154.13 111.68) (end 160.78 111.68) (width 0.25) (layer B.Cu) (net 15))
 (segment (start 153.15 110.7) (end 154.13 111.68) (width 0.25) (layer B.Cu) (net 15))
 (segment (start 160.51 113.2) (end 160.78 112.93) (width 0.25) (layer B.Cu) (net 14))
 (segment (start 153.15 113.2) (end 160.51 113.2) (width 0.25) (layer B.Cu) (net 14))
 (segment (start 109.22 115.57) (end 99.06 115.57) (width 0.25) (layer B.Cu) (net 14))
 (segment (start 115.57 109.22) (end 109.22 115.57) (width 0.25) (layer B.Cu) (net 14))
 (segment (start 144.78 109.22) (end 115.57 109.22) (width 0.25) (layer B.Cu) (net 14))
 (segment (start 148.76 113.2) (end 144.78 109.22) (width 0.25) (layer B.Cu) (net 14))
 (segment (start 153.15 113.2) (end 148.76 113.2) (width 0.25) (layer B.Cu) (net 14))
 (segment (start 141.61 107.91) (end 138.45 104.75) (width 0.5) (layer F.Cu) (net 16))
 (segment (start 141.61 113.255) (end 141.61 107.91) (width 0.5) (layer F.Cu) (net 16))
 (segment (start 160.1 92.63) (end 163.068 92.63) (width 0.5) (layer F.Cu) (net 16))
 (segment (start 151.13 101.6) (end 160.1 92.63) (width 0.5) (layer F.Cu) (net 16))
 (segment (start 147.32 101.6) (end 151.13 101.6) (width 0.5) (layer F.Cu) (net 16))
 (segment (start 141.61 107.31) (end 147.32 101.6) (width 0.5) (layer F.Cu) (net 16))
 (segment (start 141.61 107.91) (end 141.61 107.31) (width 0.5) (layer F.Cu) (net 16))
 (segment (start 101.6 114.3) (end 89.88 114.3) (width 0.25) (layer F.Cu) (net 10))
 (segment (start 89.88 114.3) (end 88.4 112.82) (width 0.25) (layer F.Cu) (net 10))
 (segment (start 107.95 120.65) (end 101.6 114.3) (width 0.25) (layer F.Cu) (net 10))
 (segment (start 121.92 120.65) (end 107.95 120.65) (width 0.25) (layer F.Cu) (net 10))
 (segment (start 99.06 113.03) (end 100.33 113.03) (width 0.25) (layer F.Cu) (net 24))
 (segment (start 100.33 113.03) (end 101.6 111.76) (width 0.25) (layer F.Cu) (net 24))
 (segment (start 101.6 110.49) (end 99.06 107.95) (width 0.25) (layer F.Cu) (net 24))
 (segment (start 101.6 111.76) (end 101.6 110.49) (width 0.25) (layer F.Cu) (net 24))
 (segment (start 93.98 88.9) (end 96.52 88.9) (width 0.5) (layer F.Cu) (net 1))
 (segment (start 82.64 88.57) (end 82.88 88.57) (width 0.5) (layer F.Cu) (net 1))
 (segment (start 91.36 88.9) (end 90.17 87.71) (width 0.5) (layer F.Cu) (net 1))
 (segment (start 93.98 88.9) (end 91.36 88.9) (width 0.5) (layer F.Cu) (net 1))
 (segment (start 84.299999 86.910001) (end 82.64 88.57) (width 0.5) (layer F.Cu) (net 1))
 (segment (start 89.370001 86.910001) (end 84.299999 86.910001) (width 0.5) (layer F.Cu) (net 1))
 (segment (start 90.17 87.71) (end 89.370001 86.910001) (width 0.5) (layer F.Cu) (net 1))
 (segment (start 87.54 88.57) (end 87.54 88.99) (width 0.25) (layer F.Cu) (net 8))
 (segment (start 87.54 88.99) (end 85.09 91.44) (width 0.25) (layer F.Cu) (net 8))
 (segment (start 85.09 91.44) (end 85.09 92.71) (width 0.25) (layer F.Cu) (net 8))
 (segment (start 85.09 92.71) (end 86.36 93.98) (width 0.25) (layer F.Cu) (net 8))
 (segment (start 86.36 93.98) (end 96.52 93.98) (width 0.25) (layer F.Cu) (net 8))
 (segment (start 87.87 91.44) (end 87.54 91.77) (width 0.5) (layer F.Cu) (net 2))
 (segment (start 89.23 91.77) (end 90.17 92.71) (width 0.5) (layer F.Cu) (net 2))
 (segment (start 87.54 91.77) (end 89.23 91.77) (width 0.5) (layer F.Cu) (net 2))
 (segment (start 92.245 92.71) (end 93.98 90.975) (width 0.5) (layer F.Cu) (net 2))
 (segment (start 90.17 92.71) (end 92.245 92.71) (width 0.5) (layer F.Cu) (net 2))
 (segment (start 93.98 90.975) (end 94.785 90.975) (width 0.5) (layer F.Cu) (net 2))
 (segment (start 95.25 91.44) (end 96.52 91.44) (width 0.5) (layer F.Cu) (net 2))
 (segment (start 94.785 90.975) (end 95.25 91.44) (width 0.5) (layer F.Cu) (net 2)))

